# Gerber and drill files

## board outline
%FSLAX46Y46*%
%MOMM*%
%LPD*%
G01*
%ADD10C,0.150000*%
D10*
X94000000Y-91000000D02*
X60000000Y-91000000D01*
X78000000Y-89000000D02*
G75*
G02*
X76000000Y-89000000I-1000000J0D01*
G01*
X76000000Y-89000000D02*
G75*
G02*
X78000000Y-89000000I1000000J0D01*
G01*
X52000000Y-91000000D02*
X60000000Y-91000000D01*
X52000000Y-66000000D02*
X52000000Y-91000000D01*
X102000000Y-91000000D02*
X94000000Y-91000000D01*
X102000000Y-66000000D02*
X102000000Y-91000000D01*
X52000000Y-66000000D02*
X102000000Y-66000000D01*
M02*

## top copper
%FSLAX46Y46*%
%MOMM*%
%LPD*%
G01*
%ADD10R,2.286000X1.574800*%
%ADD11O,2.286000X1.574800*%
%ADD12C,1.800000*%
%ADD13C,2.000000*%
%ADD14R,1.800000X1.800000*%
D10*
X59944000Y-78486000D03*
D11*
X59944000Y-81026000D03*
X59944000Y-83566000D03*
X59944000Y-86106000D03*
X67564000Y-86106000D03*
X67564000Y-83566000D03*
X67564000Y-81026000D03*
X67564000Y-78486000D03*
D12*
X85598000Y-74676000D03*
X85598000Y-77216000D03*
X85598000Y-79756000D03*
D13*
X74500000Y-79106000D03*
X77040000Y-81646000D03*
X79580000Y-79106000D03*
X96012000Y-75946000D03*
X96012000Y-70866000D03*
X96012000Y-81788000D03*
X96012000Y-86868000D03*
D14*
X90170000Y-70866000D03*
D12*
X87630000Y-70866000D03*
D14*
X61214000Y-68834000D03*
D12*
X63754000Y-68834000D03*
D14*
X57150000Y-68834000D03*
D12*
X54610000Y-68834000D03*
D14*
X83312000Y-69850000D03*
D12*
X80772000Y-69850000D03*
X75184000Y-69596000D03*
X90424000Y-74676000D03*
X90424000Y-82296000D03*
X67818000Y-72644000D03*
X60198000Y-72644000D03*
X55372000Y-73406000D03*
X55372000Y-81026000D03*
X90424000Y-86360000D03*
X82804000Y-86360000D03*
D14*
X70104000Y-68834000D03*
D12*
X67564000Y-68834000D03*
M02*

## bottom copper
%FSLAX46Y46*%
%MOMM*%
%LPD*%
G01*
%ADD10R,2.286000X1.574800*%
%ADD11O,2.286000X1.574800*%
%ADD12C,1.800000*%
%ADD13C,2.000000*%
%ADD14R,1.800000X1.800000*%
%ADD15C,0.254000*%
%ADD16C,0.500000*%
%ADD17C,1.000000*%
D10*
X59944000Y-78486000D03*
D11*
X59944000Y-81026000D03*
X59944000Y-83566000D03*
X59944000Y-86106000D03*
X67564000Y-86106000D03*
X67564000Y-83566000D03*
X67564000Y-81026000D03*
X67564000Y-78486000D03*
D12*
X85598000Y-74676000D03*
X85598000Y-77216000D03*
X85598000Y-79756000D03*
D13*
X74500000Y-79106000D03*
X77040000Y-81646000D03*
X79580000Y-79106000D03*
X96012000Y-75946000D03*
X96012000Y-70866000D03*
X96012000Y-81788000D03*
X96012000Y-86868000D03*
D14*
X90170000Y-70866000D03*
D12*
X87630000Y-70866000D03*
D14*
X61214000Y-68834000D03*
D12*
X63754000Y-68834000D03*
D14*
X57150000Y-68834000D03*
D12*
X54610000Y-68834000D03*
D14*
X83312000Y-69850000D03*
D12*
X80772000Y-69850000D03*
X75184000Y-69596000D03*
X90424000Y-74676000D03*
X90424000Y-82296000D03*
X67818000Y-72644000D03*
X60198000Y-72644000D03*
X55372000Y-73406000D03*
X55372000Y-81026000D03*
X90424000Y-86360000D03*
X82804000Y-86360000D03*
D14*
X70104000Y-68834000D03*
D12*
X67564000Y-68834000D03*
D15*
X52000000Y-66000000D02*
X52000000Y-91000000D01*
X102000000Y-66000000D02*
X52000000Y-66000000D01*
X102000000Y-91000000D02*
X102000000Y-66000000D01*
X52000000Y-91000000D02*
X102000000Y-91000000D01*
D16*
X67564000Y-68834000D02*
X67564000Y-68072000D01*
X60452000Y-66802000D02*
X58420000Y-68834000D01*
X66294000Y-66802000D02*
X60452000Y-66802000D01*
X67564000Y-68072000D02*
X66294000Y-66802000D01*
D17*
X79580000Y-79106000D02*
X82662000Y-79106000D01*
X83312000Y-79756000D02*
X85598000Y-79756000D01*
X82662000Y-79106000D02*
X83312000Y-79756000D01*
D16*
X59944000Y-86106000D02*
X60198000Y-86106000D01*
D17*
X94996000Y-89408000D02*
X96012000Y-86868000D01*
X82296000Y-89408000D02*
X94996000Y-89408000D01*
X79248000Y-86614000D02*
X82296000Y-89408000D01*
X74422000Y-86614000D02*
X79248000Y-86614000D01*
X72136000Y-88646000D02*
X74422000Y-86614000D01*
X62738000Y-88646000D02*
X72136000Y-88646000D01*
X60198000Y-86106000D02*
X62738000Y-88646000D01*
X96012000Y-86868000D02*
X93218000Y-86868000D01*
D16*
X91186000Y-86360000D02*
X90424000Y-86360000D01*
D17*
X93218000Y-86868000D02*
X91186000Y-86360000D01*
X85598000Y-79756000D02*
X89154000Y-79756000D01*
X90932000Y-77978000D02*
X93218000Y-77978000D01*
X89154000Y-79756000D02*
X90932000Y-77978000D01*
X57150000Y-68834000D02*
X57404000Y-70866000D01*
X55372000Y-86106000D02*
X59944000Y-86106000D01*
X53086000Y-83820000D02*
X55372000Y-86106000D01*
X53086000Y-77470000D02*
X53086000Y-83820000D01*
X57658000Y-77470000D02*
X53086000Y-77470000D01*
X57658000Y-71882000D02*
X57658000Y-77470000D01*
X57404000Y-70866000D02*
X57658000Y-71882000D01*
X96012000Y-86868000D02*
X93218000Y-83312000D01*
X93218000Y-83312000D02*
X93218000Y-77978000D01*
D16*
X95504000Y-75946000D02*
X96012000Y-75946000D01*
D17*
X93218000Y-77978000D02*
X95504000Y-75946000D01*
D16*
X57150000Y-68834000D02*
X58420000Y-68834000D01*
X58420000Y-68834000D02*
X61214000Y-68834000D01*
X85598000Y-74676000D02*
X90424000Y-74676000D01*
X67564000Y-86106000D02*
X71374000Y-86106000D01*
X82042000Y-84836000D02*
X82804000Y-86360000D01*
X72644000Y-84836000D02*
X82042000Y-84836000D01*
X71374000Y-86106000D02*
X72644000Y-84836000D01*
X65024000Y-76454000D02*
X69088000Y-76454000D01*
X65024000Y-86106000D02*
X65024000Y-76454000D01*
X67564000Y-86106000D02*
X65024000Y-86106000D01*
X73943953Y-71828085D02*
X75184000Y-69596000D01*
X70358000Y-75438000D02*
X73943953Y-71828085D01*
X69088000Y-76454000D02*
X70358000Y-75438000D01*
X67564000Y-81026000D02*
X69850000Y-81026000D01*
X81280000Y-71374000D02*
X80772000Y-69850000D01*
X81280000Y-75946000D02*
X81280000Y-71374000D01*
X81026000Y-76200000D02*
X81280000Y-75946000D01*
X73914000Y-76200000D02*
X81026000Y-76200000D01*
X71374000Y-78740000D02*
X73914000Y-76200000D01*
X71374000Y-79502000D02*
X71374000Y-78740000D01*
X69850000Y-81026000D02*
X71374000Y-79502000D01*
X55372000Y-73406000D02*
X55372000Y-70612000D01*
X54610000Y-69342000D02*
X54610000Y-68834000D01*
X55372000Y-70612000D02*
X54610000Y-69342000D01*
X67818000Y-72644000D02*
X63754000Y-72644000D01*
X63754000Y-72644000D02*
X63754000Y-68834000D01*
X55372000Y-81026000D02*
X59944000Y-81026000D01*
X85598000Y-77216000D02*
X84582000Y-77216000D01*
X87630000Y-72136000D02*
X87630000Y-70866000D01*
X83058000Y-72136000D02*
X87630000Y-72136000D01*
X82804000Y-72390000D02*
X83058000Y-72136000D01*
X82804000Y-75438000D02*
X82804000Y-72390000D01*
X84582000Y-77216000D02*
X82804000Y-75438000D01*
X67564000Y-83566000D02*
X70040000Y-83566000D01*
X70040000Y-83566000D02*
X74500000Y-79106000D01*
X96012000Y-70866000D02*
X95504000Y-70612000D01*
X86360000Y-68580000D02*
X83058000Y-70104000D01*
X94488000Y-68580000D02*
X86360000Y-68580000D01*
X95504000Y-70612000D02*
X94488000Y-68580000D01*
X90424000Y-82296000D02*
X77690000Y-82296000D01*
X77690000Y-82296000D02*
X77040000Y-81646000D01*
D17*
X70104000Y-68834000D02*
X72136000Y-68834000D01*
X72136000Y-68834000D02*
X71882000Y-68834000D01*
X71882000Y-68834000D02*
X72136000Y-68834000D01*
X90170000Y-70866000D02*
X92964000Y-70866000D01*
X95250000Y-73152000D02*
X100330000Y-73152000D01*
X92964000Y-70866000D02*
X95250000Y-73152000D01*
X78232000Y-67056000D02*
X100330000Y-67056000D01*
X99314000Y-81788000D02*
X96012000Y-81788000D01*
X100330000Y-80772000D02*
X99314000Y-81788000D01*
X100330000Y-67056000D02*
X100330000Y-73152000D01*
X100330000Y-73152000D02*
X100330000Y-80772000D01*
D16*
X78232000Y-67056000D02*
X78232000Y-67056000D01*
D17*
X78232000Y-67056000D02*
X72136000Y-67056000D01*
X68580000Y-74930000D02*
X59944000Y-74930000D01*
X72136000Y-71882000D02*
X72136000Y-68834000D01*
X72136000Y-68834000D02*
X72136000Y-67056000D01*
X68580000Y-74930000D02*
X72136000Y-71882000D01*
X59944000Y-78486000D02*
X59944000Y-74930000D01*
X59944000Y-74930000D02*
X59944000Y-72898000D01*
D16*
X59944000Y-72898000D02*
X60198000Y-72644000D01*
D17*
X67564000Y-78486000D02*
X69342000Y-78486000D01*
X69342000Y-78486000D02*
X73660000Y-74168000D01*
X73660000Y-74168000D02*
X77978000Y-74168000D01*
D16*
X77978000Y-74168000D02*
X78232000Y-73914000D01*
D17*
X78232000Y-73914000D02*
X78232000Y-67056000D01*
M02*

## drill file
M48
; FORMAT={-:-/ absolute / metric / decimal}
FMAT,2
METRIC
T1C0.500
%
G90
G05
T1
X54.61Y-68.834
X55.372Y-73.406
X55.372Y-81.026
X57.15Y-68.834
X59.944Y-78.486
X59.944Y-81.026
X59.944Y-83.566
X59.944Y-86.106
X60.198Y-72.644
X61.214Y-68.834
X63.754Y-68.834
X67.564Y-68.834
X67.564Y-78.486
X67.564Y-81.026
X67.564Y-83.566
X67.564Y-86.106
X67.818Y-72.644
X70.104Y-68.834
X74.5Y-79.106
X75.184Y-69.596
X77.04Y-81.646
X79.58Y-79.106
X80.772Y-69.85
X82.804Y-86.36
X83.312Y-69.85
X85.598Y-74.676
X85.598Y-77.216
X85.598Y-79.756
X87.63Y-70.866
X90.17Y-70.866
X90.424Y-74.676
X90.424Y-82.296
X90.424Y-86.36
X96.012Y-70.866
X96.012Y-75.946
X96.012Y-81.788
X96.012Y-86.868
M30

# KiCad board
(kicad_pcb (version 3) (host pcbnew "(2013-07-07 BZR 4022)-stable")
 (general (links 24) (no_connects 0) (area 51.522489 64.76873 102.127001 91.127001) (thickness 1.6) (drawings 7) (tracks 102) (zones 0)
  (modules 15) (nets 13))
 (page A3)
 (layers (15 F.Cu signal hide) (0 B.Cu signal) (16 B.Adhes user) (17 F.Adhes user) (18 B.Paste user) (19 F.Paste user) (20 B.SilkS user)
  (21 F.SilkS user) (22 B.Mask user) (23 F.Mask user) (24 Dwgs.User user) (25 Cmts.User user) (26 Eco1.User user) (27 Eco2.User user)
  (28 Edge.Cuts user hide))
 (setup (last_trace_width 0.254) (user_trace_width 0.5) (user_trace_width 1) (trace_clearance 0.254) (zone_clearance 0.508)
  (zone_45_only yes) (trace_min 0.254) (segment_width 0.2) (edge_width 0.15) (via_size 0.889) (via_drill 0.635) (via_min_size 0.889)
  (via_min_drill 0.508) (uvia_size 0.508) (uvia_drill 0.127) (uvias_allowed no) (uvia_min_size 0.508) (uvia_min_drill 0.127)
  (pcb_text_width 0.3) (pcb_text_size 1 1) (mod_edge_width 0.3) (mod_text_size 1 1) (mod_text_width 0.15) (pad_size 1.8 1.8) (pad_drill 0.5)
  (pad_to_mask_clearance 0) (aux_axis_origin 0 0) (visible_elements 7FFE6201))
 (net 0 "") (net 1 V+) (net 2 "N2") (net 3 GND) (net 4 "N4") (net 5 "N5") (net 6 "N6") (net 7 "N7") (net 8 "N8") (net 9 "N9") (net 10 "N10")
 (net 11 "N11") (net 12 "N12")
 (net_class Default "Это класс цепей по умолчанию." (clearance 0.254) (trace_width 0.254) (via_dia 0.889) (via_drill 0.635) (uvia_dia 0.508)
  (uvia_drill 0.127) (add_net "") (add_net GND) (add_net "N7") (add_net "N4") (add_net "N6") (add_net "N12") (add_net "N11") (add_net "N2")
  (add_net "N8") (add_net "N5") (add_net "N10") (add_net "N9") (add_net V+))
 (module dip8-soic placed (layer F.Cu) (at 63.754 82.296 270)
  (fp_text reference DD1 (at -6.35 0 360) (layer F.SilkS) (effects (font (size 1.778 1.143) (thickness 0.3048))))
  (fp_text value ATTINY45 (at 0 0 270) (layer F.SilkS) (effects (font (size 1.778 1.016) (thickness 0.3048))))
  (pad 1 thru_hole rect (at -3.81 3.81 270) (size 1.5748 2.286) (drill 0.5) (layers *.Cu *.Mask F.SilkS) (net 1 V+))
  (pad 2 thru_hole oval (at -1.27 3.81 270) (size 1.5748 2.286) (drill 0.5) (layers *.Cu *.Mask F.SilkS) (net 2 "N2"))
  (pad 3 thru_hole oval (at 1.27 3.81 270) (size 1.5748 2.286) (drill 0.5) (layers *.Cu *.Mask F.SilkS))
  (pad 4 thru_hole oval (at 3.81 3.81 270) (size 1.5748 2.286) (drill 0.5) (layers *.Cu *.Mask F.SilkS) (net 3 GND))
  (pad 5 thru_hole oval (at 3.81 -3.81 270) (size 1.5748 2.286) (drill 0.5) (layers *.Cu *.Mask F.SilkS) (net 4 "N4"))
  (pad 6 thru_hole oval (at 1.27 -3.81 270) (size 1.5748 2.286) (drill 0.5) (layers *.Cu *.Mask F.SilkS) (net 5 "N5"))
  (pad 7 thru_hole oval (at -1.27 -3.81 270) (size 1.5748 2.286) (drill 0.5) (layers *.Cu *.Mask F.SilkS) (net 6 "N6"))
  (pad 8 thru_hole oval (at -3.81 -3.81 270) (size 1.5748 2.286) (drill 0.5) (layers *.Cu *.Mask F.SilkS) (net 1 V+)))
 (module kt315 (layer F.Cu) (at 85.598 77.216 90)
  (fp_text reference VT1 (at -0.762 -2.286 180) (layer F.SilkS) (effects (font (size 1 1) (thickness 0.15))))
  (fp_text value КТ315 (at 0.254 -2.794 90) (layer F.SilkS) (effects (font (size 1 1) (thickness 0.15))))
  (pad 1 thru_hole circle (at 2.54 0 90) (size 1.8 1.8) (drill 0.5) (layers *.Cu *.Mask F.SilkS) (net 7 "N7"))
  (pad 2 thru_hole circle (at 0 0 90) (size 1.8 1.8) (drill 0.5) (layers *.Cu *.Mask F.SilkS) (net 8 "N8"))
  (pad 3 thru_hole circle (at -2.54 0 90) (size 1.8 1.8) (drill 0.5) (layers *.Cu *.Mask F.SilkS) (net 3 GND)))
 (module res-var (layer F.Cu) (at 76.454 79.502) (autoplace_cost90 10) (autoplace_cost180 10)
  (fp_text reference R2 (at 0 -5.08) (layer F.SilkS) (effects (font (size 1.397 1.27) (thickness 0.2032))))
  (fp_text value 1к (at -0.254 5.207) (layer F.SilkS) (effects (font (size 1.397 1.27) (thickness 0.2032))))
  (pad 1 thru_hole circle (at -1.954 -0.396) (size 2 2) (drill 0.5) (layers *.Cu *.Mask F.SilkS) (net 5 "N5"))
  (pad 2 thru_hole circle (at 0.586 2.144) (size 2 2) (drill 0.5) (layers *.Cu *.Mask F.SilkS) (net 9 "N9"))
  (pad 3 thru_hole circle (at 3.126 -0.396) (size 2 2) (drill 0.5) (layers *.Cu *.Mask F.SilkS) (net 3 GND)))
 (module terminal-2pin (layer F.Cu) (at 96.012 73.406 90)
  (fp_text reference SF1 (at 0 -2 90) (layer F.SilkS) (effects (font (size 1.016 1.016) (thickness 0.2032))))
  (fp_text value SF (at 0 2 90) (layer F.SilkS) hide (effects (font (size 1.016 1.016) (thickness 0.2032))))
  (pad 1 thru_hole circle (at -2.54 0 90) (size 2 2) (drill 0.5) (layers *.Cu *.Mask F.SilkS) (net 3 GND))
  (pad 2 thru_hole circle (at 2.54 0 90) (size 2 2) (drill 0.5) (layers *.Cu *.Mask F.SilkS) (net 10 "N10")))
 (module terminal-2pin (layer F.Cu) (at 96.012 84.328 270)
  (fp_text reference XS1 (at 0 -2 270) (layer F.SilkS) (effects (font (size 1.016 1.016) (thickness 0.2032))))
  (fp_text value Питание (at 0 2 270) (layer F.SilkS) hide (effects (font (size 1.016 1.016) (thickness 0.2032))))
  (pad 1 thru_hole circle (at -2.54 0 270) (size 2 2) (drill 0.5) (layers *.Cu *.Mask F.SilkS) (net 1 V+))
  (pad 2 thru_hole circle (at 2.54 0 270) (size 2 2) (drill 0.5) (layers *.Cu *.Mask F.SilkS) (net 3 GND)))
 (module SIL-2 (layer F.Cu) (at 88.9 70.866 180)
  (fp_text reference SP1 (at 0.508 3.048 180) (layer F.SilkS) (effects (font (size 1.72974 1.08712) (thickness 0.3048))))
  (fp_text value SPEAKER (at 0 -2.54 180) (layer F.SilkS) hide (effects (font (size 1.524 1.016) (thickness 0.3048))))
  (pad 1 thru_hole rect (at -1.27 0 180) (size 1.8 1.8) (drill 0.5) (layers *.Cu *.Mask F.SilkS) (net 1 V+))
  (pad 2 thru_hole circle (at 1.27 0 180) (size 1.8 1.8) (drill 0.5) (layers *.Cu *.Mask F.SilkS) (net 8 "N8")))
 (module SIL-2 (layer F.Cu) (at 62.484 68.834)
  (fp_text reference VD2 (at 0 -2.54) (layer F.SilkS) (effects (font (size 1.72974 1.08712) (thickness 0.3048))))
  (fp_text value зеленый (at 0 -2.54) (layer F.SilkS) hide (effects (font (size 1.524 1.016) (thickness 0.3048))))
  (pad 1 thru_hole rect (at -1.27 0) (size 1.8 1.8) (drill 0.5) (layers *.Cu *.Mask F.SilkS) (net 3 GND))
  (pad 2 thru_hole circle (at 1.27 0) (size 1.8 1.8) (drill 0.5) (layers *.Cu *.Mask F.SilkS) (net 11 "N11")))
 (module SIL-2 (layer F.Cu) (at 55.88 68.834 180)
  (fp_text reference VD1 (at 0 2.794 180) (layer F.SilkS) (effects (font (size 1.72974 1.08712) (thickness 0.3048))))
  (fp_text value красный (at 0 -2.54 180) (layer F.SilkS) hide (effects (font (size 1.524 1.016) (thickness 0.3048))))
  (pad 1 thru_hole rect (at -1.27 0 180) (size 1.8 1.8) (drill 0.5) (layers *.Cu *.Mask F.SilkS) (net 3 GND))
  (pad 2 thru_hole circle (at 1.27 0 180) (size 1.8 1.8) (drill 0.5) (layers *.Cu *.Mask F.SilkS) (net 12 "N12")))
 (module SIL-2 (layer F.Cu) (at 82.042 69.85 180)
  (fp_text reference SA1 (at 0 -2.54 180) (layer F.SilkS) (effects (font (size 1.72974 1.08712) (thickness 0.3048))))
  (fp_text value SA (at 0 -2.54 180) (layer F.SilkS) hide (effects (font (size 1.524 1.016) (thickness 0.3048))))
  (pad 1 thru_hole rect (at -1.27 0 180) (size 1.8 1.8) (drill 0.5) (layers *.Cu *.Mask F.SilkS) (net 10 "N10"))
  (pad 2 thru_hole circle (at 1.27 0 180) (size 1.8 1.8) (drill 0.5) (layers *.Cu *.Mask F.SilkS) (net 6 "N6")))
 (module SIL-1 (layer F.Cu) (at 75.184 69.596)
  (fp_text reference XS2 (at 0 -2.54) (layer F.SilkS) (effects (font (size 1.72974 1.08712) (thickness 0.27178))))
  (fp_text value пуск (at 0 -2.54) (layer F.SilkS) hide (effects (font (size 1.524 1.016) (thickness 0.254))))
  (pad 1 thru_hole circle (at 0 0) (size 1.8 1.8) (drill 0.5) (layers *.Cu *.Mask F.SilkS) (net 4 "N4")))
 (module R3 (layer F.Cu) (at 90.424 78.486 270) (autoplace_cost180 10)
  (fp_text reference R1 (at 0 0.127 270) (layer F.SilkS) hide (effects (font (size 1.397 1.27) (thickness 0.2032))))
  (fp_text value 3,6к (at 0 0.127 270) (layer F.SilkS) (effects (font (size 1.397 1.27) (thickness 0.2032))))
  (pad 1 thru_hole circle (at -3.81 0 270) (size 1.8 1.8) (drill 0.5) (layers *.Cu *.Mask F.SilkS) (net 7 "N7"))
  (pad 2 thru_hole circle (at 3.81 0 270) (size 1.8 1.8) (drill 0.5) (layers *.Cu *.Mask F.SilkS) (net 9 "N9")))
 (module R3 (layer F.Cu) (at 64.008 72.644 180) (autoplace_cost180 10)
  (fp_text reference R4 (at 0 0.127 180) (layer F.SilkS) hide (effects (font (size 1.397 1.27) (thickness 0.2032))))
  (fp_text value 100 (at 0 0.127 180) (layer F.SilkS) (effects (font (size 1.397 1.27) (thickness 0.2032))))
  (pad 1 thru_hole circle (at -3.81 0 180) (size 1.8 1.8) (drill 0.5) (layers *.Cu *.Mask F.SilkS) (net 11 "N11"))
  (pad 2 thru_hole circle (at 3.81 0 180) (size 1.8 1.8) (drill 0.5) (layers *.Cu *.Mask F.SilkS) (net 1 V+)))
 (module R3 (layer F.Cu) (at 55.372 77.216 270) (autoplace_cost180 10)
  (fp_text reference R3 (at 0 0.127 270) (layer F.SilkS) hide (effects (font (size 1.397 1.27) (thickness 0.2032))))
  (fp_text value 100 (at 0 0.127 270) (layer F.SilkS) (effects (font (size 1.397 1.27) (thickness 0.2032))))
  (pad 1 thru_hole circle (at -3.81 0 270) (size 1.8 1.8) (drill 0.5) (layers *.Cu *.Mask F.SilkS) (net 12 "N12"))
  (pad 2 thru_hole circle (at 3.81 0 270) (size 1.8 1.8) (drill 0.5) (layers *.Cu *.Mask F.SilkS) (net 2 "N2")))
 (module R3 (layer F.Cu) (at 86.614 86.36 180) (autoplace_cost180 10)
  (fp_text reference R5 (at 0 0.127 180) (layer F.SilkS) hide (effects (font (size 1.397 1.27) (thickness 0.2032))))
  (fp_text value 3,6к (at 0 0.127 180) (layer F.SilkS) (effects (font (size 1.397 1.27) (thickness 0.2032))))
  (pad 1 thru_hole circle (at -3.81 0 180) (size 1.8 1.8) (drill 0.5) (layers *.Cu *.Mask F.SilkS) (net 3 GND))
  (pad 2 thru_hole circle (at 3.81 0 180) (size 1.8 1.8) (drill 0.5) (layers *.Cu *.Mask F.SilkS) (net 4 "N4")))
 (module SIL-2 (layer F.Cu) (at 68.834 68.834 180)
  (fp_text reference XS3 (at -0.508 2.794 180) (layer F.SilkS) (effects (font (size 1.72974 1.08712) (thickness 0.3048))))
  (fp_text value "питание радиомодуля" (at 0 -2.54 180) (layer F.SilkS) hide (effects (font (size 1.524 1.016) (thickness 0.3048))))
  (pad 1 thru_hole rect (at -1.27 0 180) (size 1.8 1.8) (drill 0.5) (layers *.Cu *.Mask F.SilkS) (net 1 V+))
  (pad 2 thru_hole circle (at 1.27 0 180) (size 1.8 1.8) (drill 0.5) (layers *.Cu *.Mask F.SilkS) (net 3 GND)))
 (gr_line (start 94 91) (end 60 91) (angle 90) (layer Edge.Cuts) (width 0.15))
 (gr_circle (center 77 89) (end 77 88) (layer Edge.Cuts) (width 0.15))
 (gr_line (start 52 91) (end 60 91) (angle 90) (layer Edge.Cuts) (width 0.15))
 (gr_line (start 52 66) (end 52 91) (angle 90) (layer Edge.Cuts) (width 0.15))
 (gr_line (start 102 91) (end 94 91) (angle 90) (layer Edge.Cuts) (width 0.15))
 (gr_line (start 102 66) (end 102 91) (angle 90) (layer Edge.Cuts) (width 0.15))
 (gr_line (start 52 66) (end 102 66) (angle 90) (layer Edge.Cuts) (width 0.15))
 (segment (start 52 66) (end 52 91) (width 0.254) (layer B.Cu) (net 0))
 (segment (start 102 66) (end 52 66) (width 0.254) (layer B.Cu) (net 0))
 (segment (start 102 91) (end 102 66) (width 0.254) (layer B.Cu) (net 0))
 (segment (start 52 91) (end 102 91) (width 0.254) (layer B.Cu) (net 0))
 (segment (start 67.564 68.834) (end 67.564 68.072) (width 0.5) (layer B.Cu) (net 3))
 (segment (start 60.452 66.802) (end 58.42 68.834) (width 0.5) (layer B.Cu) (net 3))
 (segment (start 66.294 66.802) (end 60.452 66.802) (width 0.5) (layer B.Cu) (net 3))
 (segment (start 67.564 68.072) (end 66.294 66.802) (width 0.5) (layer B.Cu) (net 3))
 (segment (start 79.58 79.106) (end 82.662 79.106) (width 1) (layer B.Cu) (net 3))
 (segment (start 83.312 79.756) (end 85.598 79.756) (width 1) (layer B.Cu) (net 3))
 (segment (start 82.662 79.106) (end 83.312 79.756) (width 1) (layer B.Cu) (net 3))
 (segment (start 59.944 86.106) (end 60.198 86.106) (width 0.5) (layer B.Cu) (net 3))
 (segment (start 94.996 89.408) (end 96.012 86.868) (width 1) (layer B.Cu) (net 3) (status 20))
 (segment (start 82.296 89.408) (end 94.996 89.408) (width 1) (layer B.Cu) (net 3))
 (segment (start 79.248 86.614) (end 82.296 89.408) (width 1) (layer B.Cu) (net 3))
 (segment (start 74.422 86.614) (end 79.248 86.614) (width 1) (layer B.Cu) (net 3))
 (segment (start 72.136 88.646) (end 74.422 86.614) (width 1) (layer B.Cu) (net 3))
 (segment (start 62.738 88.646) (end 72.136 88.646) (width 1) (layer B.Cu) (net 3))
 (segment (start 60.198 86.106) (end 62.738 88.646) (width 1) (layer B.Cu) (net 3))
 (segment (start 96.012 86.868) (end 93.218 86.868) (width 1) (layer B.Cu) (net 3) (status 10))
 (segment (start 91.186 86.36) (end 90.424 86.36) (width 0.5) (layer B.Cu) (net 3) (status 30))
 (segment (start 93.218 86.868) (end 91.186 86.36) (width 1) (layer B.Cu) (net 3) (status 20))
 (segment (start 85.598 79.756) (end 89.154 79.756) (width 1) (layer B.Cu) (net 3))
 (segment (start 90.932 77.978) (end 93.218 77.978) (width 1) (layer B.Cu) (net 3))
 (segment (start 89.154 79.756) (end 90.932 77.978) (width 1) (layer B.Cu) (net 3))
 (segment (start 57.15 68.834) (end 57.404 70.866) (width 1) (layer B.Cu) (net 3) (status 10))
 (segment (start 55.372 86.106) (end 59.944 86.106) (width 1) (layer B.Cu) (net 3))
 (segment (start 53.086 83.82) (end 55.372 86.106) (width 1) (layer B.Cu) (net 3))
 (segment (start 53.086 77.47) (end 53.086 83.82) (width 1) (layer B.Cu) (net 3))
 (segment (start 57.658 77.47) (end 53.086 77.47) (width 1) (layer B.Cu) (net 3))
 (segment (start 57.658 71.882) (end 57.658 77.47) (width 1) (layer B.Cu) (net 3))
 (segment (start 57.404 70.866) (end 57.658 71.882) (width 1) (layer B.Cu) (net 3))
 (segment (start 96.012 86.868) (end 93.218 83.312) (width 1) (layer B.Cu) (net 3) (status 10))
 (segment (start 93.218 83.312) (end 93.218 77.978) (width 1) (layer B.Cu) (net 3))
 (segment (start 95.504 75.946) (end 96.012 75.946) (width 0.5) (layer B.Cu) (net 3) (status 30))
 (segment (start 93.218 77.978) (end 95.504 75.946) (width 1) (layer B.Cu) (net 3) (status 20))
 (segment (start 57.15 68.834) (end 58.42 68.834) (width 0.5) (layer B.Cu) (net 3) (status 20))
 (segment (start 58.42 68.834) (end 61.214 68.834) (width 0.5) (layer B.Cu) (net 3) (status 20))
 (segment (start 85.598 74.676) (end 90.424 74.676) (width 0.5) (layer B.Cu) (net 7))
 (segment (start 67.564 86.106) (end 71.374 86.106) (width 0.5) (layer B.Cu) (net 4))
 (segment (start 82.042 84.836) (end 82.804 86.36) (width 0.5) (layer B.Cu) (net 4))
 (segment (start 72.644 84.836) (end 82.042 84.836) (width 0.5) (layer B.Cu) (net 4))
 (segment (start 71.374 86.106) (end 72.644 84.836) (width 0.5) (layer B.Cu) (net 4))
 (segment (start 65.024 76.454) (end 69.088 76.454) (width 0.5) (layer B.Cu) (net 4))
 (segment (start 65.024 86.106) (end 65.024 76.454) (width 0.5) (layer B.Cu) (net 4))
 (segment (start 67.564 86.106) (end 65.024 86.106) (width 0.5) (layer B.Cu) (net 4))
 (segment (start 73.943953 71.828085) (end 75.184 69.596) (width 0.5) (layer B.Cu) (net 4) (status 20))
 (segment (start 70.358 75.438) (end 73.943953 71.828085) (width 0.5) (layer B.Cu) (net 4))
 (segment (start 69.088 76.454) (end 70.358 75.438) (width 0.5) (layer B.Cu) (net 4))
 (segment (start 67.564 81.026) (end 69.85 81.026) (width 0.5) (layer B.Cu) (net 6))
 (segment (start 81.28 71.374) (end 80.772 69.85) (width 0.5) (layer B.Cu) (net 6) (status 20))
 (segment (start 81.28 75.946) (end 81.28 71.374) (width 0.5) (layer B.Cu) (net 6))
 (segment (start 81.026 76.2) (end 81.28 75.946) (width 0.5) (layer B.Cu) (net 6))
 (segment (start 73.914 76.2) (end 81.026 76.2) (width 0.5) (layer B.Cu) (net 6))
 (segment (start 71.374 78.74) (end 73.914 76.2) (width 0.5) (layer B.Cu) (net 6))
 (segment (start 71.374 79.502) (end 71.374 78.74) (width 0.5) (layer B.Cu) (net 6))
 (segment (start 69.85 81.026) (end 71.374 79.502) (width 0.5) (layer B.Cu) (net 6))
 (segment (start 55.372 73.406) (end 55.372 70.612) (width 0.5) (layer B.Cu) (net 12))
 (segment (start 54.61 69.342) (end 54.61 68.834) (width 0.5) (layer B.Cu) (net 12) (status 30))
 (segment (start 55.372 70.612) (end 54.61 69.342) (width 0.5) (layer B.Cu) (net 12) (status 20))
 (segment (start 67.818 72.644) (end 63.754 72.644) (width 0.5) (layer B.Cu) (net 11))
 (segment (start 63.754 72.644) (end 63.754 68.834) (width 0.5) (layer B.Cu) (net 11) (status 20))
 (segment (start 55.372 81.026) (end 59.944 81.026) (width 0.5) (layer B.Cu) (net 2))
 (segment (start 85.598 77.216) (end 84.582 77.216) (width 0.5) (layer B.Cu) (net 8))
 (segment (start 87.63 72.136) (end 87.63 70.866) (width 0.5) (layer B.Cu) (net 8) (status 20))
 (segment (start 83.058 72.136) (end 87.63 72.136) (width 0.5) (layer B.Cu) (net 8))
 (segment (start 82.804 72.39) (end 83.058 72.136) (width 0.5) (layer B.Cu) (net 8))
 (segment (start 82.804 75.438) (end 82.804 72.39) (width 0.5) (layer B.Cu) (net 8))
 (segment (start 84.582 77.216) (end 82.804 75.438) (width 0.5) (layer B.Cu) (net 8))
 (segment (start 67.564 83.566) (end 70.04 83.566) (width 0.5) (layer B.Cu) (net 5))
 (segment (start 70.04 83.566) (end 74.5 79.106) (width 0.5) (layer B.Cu) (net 5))
 (segment (start 96.012 70.866) (end 95.504 70.612) (width 0.5) (layer B.Cu) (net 10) (status 10))
 (segment (start 86.36 68.58) (end 83.058 70.104) (width 0.5) (layer B.Cu) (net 10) (status 20))
 (segment (start 94.488 68.58) (end 86.36 68.58) (width 0.5) (layer B.Cu) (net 10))
 (segment (start 95.504 70.612) (end 94.488 68.58) (width 0.5) (layer B.Cu) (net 10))
 (segment (start 90.424 82.296) (end 77.69 82.296) (width 0.5) (layer B.Cu) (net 9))
 (segment (start 77.69 82.296) (end 77.04 81.646) (width 0.5) (layer B.Cu) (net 9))
 (segment (start 70.104 68.834) (end 72.136 68.834) (width 1) (layer B.Cu) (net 1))
 (segment (start 72.136 68.834) (end 71.882 68.834) (width 1) (layer B.Cu) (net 1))
 (segment (start 71.882 68.834) (end 72.136 68.834) (width 1) (layer B.Cu) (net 1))
 (segment (start 90.17 70.866) (end 92.964 70.866) (width 1) (layer B.Cu) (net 1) (status 10))
 (segment (start 95.25 73.152) (end 100.33 73.152) (width 1) (layer B.Cu) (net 1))
 (segment (start 92.964 70.866) (end 95.25 73.152) (width 1) (layer B.Cu) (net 1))
 (segment (start 78.232 67.056) (end 100.33 67.056) (width 1) (layer B.Cu) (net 1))
 (segment (start 99.314 81.788) (end 96.012 81.788) (width 1) (layer B.Cu) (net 1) (status 20))
 (segment (start 100.33 80.772) (end 99.314 81.788) (width 1) (layer B.Cu) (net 1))
 (segment (start 100.33 67.056) (end 100.33 73.152) (width 1) (layer B.Cu) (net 1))
 (segment (start 100.33 73.152) (end 100.33 80.772) (width 1) (layer B.Cu) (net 1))
 (segment (start 78.232 67.056) (end 78.232 67.056) (width 0.5) (layer B.Cu) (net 1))
 (segment (start 78.232 67.056) (end 72.136 67.056) (width 1) (layer B.Cu) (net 1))
 (segment (start 68.58 74.93) (end 59.944 74.93) (width 1) (layer B.Cu) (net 1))
 (segment (start 72.136 71.882) (end 72.136 68.834) (width 1) (layer B.Cu) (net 1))
 (segment (start 72.136 68.834) (end 72.136 67.056) (width 1) (layer B.Cu) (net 1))
 (segment (start 68.58 74.93) (end 72.136 71.882) (width 1) (layer B.Cu) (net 1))
 (segment (start 59.944 78.486) (end 59.944 74.93) (width 1) (layer B.Cu) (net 1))
 (segment (start 59.944 74.93) (end 59.944 72.898) (width 1) (layer B.Cu) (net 1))
 (segment (start 59.944 72.898) (end 60.198 72.644) (width 0.5) (layer B.Cu) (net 1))
 (segment (start 67.564 78.486) (end 69.342 78.486) (width 1) (layer B.Cu) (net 1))
 (segment (start 69.342 78.486) (end 73.66 74.168) (width 1) (layer B.Cu) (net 1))
 (segment (start 73.66 74.168) (end 77.978 74.168) (width 1) (layer B.Cu) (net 1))
 (segment (start 77.978 74.168) (end 78.232 73.914) (width 0.5) (layer B.Cu) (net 1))
 (segment (start 78.232 73.914) (end 78.232 67.056) (width 1) (layer B.Cu) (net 1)))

